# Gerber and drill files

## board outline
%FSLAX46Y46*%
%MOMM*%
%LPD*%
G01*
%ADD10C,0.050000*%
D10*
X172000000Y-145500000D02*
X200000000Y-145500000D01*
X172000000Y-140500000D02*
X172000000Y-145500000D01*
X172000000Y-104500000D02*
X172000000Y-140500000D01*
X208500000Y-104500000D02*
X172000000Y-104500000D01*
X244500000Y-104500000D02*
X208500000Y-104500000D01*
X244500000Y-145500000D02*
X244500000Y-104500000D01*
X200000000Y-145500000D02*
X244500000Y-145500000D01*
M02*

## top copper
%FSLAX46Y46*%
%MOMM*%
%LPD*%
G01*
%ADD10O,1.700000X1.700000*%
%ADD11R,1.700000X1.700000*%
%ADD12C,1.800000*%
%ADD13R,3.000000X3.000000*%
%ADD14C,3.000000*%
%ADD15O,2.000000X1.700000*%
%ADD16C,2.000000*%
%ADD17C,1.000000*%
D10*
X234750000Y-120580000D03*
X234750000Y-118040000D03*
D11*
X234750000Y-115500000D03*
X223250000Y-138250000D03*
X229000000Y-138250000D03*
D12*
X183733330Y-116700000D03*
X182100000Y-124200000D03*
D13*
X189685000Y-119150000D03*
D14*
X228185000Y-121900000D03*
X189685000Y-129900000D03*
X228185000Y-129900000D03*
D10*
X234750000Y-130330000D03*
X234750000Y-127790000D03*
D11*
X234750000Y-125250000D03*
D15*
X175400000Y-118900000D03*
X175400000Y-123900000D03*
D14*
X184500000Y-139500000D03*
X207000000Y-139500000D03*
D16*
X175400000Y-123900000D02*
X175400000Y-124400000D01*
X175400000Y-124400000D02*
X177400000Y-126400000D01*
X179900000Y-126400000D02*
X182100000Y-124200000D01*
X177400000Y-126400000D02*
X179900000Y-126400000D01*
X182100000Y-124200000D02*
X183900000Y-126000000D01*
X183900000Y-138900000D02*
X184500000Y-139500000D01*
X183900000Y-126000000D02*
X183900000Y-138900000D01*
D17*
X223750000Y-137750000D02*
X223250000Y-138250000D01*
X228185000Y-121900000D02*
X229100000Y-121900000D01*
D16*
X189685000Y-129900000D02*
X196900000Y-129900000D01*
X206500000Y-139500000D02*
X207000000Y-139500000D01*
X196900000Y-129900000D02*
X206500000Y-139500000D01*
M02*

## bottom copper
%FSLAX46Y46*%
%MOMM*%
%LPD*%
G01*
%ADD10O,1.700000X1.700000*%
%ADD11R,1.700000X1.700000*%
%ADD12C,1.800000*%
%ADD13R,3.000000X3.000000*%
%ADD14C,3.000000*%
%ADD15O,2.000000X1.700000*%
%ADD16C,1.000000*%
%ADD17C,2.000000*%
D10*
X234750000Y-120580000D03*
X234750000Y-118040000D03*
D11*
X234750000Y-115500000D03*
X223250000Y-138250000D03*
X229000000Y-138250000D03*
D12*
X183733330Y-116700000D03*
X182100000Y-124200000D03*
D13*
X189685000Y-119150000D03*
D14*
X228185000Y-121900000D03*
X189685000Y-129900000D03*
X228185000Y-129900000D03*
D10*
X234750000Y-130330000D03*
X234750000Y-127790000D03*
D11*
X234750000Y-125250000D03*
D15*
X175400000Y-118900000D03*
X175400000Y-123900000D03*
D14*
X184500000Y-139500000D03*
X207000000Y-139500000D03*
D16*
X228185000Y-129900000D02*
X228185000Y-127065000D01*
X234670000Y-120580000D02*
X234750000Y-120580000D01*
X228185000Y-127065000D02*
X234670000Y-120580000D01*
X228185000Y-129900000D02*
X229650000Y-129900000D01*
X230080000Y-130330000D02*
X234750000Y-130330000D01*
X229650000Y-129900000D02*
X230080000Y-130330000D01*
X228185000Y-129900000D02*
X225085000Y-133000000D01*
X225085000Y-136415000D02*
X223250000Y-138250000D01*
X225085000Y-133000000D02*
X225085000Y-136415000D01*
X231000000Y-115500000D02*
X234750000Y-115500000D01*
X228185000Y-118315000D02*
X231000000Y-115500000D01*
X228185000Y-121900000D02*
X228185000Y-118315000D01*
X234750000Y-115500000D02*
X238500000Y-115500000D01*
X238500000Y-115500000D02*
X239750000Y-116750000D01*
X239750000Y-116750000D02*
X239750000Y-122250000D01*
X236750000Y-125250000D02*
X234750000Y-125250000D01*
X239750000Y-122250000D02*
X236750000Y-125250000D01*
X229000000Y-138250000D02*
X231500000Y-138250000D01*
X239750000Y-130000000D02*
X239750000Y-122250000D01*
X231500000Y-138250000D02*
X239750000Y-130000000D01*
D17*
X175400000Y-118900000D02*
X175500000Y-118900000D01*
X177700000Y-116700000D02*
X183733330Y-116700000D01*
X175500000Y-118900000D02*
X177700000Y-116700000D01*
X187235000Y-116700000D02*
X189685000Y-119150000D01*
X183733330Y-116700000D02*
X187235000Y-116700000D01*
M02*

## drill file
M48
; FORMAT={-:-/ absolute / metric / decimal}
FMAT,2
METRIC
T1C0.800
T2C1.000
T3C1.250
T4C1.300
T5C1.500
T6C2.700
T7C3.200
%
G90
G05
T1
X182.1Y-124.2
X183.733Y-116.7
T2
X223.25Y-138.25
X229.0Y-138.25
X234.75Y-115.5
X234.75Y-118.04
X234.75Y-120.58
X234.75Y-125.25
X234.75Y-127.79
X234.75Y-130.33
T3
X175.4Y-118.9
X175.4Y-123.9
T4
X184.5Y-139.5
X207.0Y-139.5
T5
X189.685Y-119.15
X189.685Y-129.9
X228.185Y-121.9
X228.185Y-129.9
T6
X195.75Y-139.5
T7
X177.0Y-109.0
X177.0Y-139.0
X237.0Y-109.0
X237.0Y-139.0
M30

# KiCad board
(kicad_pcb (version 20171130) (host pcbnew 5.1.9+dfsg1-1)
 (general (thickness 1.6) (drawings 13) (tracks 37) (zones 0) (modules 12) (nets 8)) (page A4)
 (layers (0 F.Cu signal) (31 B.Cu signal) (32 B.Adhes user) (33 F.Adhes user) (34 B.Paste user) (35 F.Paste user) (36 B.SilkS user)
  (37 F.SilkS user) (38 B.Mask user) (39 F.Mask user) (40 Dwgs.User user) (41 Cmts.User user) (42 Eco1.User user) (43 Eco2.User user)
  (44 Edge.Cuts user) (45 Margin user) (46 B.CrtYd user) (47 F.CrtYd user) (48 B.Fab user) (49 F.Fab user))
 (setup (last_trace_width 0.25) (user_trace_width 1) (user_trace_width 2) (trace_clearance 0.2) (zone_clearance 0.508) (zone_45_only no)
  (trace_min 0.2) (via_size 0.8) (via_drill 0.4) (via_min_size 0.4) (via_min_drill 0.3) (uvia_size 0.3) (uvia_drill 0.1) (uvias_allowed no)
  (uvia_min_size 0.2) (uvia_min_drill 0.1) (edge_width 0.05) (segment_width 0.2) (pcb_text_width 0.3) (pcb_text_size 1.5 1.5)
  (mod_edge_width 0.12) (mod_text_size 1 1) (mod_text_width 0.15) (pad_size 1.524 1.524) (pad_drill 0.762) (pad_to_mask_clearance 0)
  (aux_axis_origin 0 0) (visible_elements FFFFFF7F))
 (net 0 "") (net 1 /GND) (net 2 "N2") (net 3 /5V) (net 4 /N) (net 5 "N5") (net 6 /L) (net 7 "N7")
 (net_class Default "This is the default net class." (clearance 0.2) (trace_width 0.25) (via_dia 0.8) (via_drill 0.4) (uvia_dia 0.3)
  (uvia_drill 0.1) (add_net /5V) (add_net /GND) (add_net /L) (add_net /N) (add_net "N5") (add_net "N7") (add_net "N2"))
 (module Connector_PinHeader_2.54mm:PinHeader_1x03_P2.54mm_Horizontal (layer F.Cu) (at 234.75 115.5)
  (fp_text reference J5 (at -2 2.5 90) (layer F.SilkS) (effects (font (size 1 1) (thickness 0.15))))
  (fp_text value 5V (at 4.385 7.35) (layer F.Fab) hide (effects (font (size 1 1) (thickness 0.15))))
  (pad 3 thru_hole oval (at 0 5.08) (size 1.7 1.7) (drill 1) (layers *.Cu *.Mask) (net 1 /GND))
  (pad 2 thru_hole oval (at 0 2.54) (size 1.7 1.7) (drill 1) (layers *.Cu *.Mask) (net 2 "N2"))
  (pad 1 thru_hole rect (at 0 0) (size 1.7 1.7) (drill 1) (layers *.Cu *.Mask) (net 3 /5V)))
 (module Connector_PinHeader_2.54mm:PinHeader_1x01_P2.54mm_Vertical (layer F.Cu) (at 223.25 138.25)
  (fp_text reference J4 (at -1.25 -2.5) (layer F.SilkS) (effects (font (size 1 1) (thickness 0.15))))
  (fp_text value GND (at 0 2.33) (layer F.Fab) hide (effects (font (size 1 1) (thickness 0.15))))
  (pad 1 thru_hole rect (at 0 0) (size 1.7 1.7) (drill 1) (layers *.Cu *.Mask) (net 1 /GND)))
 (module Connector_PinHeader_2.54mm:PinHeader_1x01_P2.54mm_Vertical (layer F.Cu) (at 229 138.25)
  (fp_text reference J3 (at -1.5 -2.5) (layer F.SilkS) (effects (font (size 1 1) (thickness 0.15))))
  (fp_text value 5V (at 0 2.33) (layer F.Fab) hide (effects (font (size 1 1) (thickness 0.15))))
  (pad 1 thru_hole rect (at 0 0) (size 1.7 1.7) (drill 1) (layers *.Cu *.Mask) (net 3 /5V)))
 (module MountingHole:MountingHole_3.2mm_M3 (layer F.Cu) (at 237 109)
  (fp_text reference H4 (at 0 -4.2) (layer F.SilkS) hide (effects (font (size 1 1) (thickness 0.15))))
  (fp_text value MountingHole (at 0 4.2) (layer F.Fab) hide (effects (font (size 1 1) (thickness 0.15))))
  (pad 1 np_thru_hole circle (at 0 0) (size 3.2 3.2) (drill 3.2) (layers *.Cu *.Mask)))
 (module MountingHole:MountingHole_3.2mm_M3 (layer F.Cu) (at 237 139)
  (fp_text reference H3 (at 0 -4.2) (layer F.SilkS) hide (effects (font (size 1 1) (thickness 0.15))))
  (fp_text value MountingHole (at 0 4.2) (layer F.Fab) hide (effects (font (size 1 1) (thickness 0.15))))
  (pad 1 np_thru_hole circle (at 0 0) (size 3.2 3.2) (drill 3.2) (layers *.Cu *.Mask)))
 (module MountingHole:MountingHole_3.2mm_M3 (layer F.Cu) (at 177 109)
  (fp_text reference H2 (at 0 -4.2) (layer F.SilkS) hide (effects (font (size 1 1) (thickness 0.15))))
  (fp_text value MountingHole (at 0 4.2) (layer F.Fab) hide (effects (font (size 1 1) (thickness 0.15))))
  (pad 1 np_thru_hole circle (at 0 0) (size 3.2 3.2) (drill 3.2) (layers *.Cu *.Mask)))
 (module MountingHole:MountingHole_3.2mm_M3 (layer F.Cu) (at 177 139)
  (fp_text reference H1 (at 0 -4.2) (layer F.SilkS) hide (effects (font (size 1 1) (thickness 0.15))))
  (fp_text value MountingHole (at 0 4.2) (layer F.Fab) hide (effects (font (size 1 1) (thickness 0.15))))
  (pad 1 np_thru_hole circle (at 0 0) (size 3.2 3.2) (drill 3.2) (layers *.Cu *.Mask)))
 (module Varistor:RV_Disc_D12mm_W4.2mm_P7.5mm (layer F.Cu) (at 182.1 124.2 90)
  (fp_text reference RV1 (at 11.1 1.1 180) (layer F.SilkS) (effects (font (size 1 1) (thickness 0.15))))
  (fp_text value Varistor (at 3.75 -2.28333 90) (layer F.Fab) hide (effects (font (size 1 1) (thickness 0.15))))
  (pad 2 thru_hole circle (at 7.5 1.63333 90) (size 1.8 1.8) (drill 0.8) (layers *.Cu *.Mask) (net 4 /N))
  (pad 1 thru_hole circle (at 0 0 90) (size 1.8 1.8) (drill 0.8) (layers *.Cu *.Mask) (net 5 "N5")))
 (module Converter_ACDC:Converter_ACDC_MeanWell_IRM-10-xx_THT (layer F.Cu) (at 189.685 119.15)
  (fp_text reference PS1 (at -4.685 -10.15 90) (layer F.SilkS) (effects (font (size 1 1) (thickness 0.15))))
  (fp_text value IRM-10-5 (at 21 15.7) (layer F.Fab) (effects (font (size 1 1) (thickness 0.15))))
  (pad 1 thru_hole rect (at 0 0) (size 3 3) (drill 1.5) (layers *.Cu *.Mask) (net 4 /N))
  (pad 4 thru_hole circle (at 38.5 2.75) (size 3 3) (drill 1.5) (layers *.Cu *.Mask) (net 3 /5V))
  (pad 2 thru_hole circle (at 0 10.75) (size 3 3) (drill 1.5) (layers *.Cu *.Mask) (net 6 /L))
  (pad 3 thru_hole circle (at 38.5 10.75) (size 3 3) (drill 1.5) (layers *.Cu *.Mask) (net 1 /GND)))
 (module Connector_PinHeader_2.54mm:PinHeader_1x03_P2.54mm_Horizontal (layer F.Cu) (at 234.75 125.25)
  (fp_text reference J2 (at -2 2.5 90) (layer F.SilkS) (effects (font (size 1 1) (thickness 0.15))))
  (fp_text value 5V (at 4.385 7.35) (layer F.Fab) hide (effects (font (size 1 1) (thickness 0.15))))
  (pad 3 thru_hole oval (at 0 5.08) (size 1.7 1.7) (drill 1) (layers *.Cu *.Mask) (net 1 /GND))
  (pad 2 thru_hole oval (at 0 2.54) (size 1.7 1.7) (drill 1) (layers *.Cu *.Mask) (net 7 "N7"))
  (pad 1 thru_hole rect (at 0 0) (size 1.7 1.7) (drill 1) (layers *.Cu *.Mask) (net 3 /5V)))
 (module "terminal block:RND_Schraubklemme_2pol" (layer F.Cu) (at 175.4 118.9 270)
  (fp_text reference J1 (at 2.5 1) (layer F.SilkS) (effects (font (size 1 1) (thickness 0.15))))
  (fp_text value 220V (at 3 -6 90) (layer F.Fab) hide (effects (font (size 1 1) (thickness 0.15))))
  (pad 1 thru_hole oval (at 0 0 270) (size 1.7 2) (drill 1.25) (layers *.Cu *.Mask) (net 4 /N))
  (pad 2 thru_hole oval (at 5 0 270) (size 1.7 2) (drill 1.25) (layers *.Cu *.Mask) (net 5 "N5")))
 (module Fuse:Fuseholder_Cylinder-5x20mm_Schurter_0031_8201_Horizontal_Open (layer F.Cu) (at 207 139.5 180)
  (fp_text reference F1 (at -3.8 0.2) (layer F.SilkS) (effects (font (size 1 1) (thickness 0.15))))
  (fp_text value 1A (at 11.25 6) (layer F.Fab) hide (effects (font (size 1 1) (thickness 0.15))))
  (pad "" np_thru_hole circle (at 11.25 0 180) (size 2.7 2.7) (drill 2.7) (layers *.Cu *.Mask))
  (pad 2 thru_hole circle (at 22.5 0 180) (size 3 3) (drill 1.3) (layers *.Cu *.Mask) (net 5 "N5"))
  (pad 1 thru_hole circle (at 0 0 180) (size 3 3) (drill 1.3) (layers *.Cu *.Mask) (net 6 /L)))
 (gr_line (start 172 145.5) (end 200 145.5) (layer Edge.Cuts) (width 0.05))
 (gr_line (start 172 140.5) (end 172 145.5) (layer Edge.Cuts) (width 0.05))
 (gr_line (start 172 104.5) (end 172 140.5) (layer Edge.Cuts) (width 0.05))
 (gr_line (start 208.5 104.5) (end 172 104.5) (layer Edge.Cuts) (width 0.05))
 (gr_line (start 244.5 104.5) (end 208.5 104.5) (layer Edge.Cuts) (width 0.05))
 (gr_line (start 244.5 145.5) (end 244.5 104.5) (layer Edge.Cuts) (width 0.05))
 (gr_line (start 200 145.5) (end 244.5 145.5) (layer Edge.Cuts) (width 0.05))
 (segment (start 175.4 123.9) (end 175.4 124.4) (width 2) (layer F.Cu) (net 5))
 (segment (start 175.4 124.4) (end 177.4 126.4) (width 2) (layer F.Cu) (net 5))
 (segment (start 179.9 126.4) (end 182.1 124.2) (width 2) (layer F.Cu) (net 5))
 (segment (start 177.4 126.4) (end 179.9 126.4) (width 2) (layer F.Cu) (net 5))
 (segment (start 182.1 124.2) (end 183.9 126) (width 2) (layer F.Cu) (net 5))
 (segment (start 183.9 138.9) (end 184.5 139.5) (width 2) (layer F.Cu) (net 5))
 (segment (start 183.9 126) (end 183.9 138.9) (width 2) (layer F.Cu) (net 5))
 (segment (start 223.75 137.75) (end 223.25 138.25) (width 1) (layer F.Cu) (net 1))
 (segment (start 228.185 129.9) (end 228.185 127.065) (width 1) (layer B.Cu) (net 1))
 (segment (start 234.67 120.58) (end 234.75 120.58) (width 1) (layer B.Cu) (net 1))
 (segment (start 228.185 127.065) (end 234.67 120.58) (width 1) (layer B.Cu) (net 1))
 (segment (start 228.185 129.9) (end 229.65 129.9) (width 1) (layer B.Cu) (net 1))
 (segment (start 230.08 130.33) (end 234.75 130.33) (width 1) (layer B.Cu) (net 1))
 (segment (start 229.65 129.9) (end 230.08 130.33) (width 1) (layer B.Cu) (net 1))
 (segment (start 228.185 129.9) (end 225.085 133) (width 1) (layer B.Cu) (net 1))
 (segment (start 225.085 136.415) (end 223.25 138.25) (width 1) (layer B.Cu) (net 1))
 (segment (start 225.085 133) (end 225.085 136.415) (width 1) (layer B.Cu) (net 1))
 (segment (start 228.185 121.9) (end 229.1 121.9) (width 1) (layer F.Cu) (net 3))
 (segment (start 231 115.5) (end 234.75 115.5) (width 1) (layer B.Cu) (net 3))
 (segment (start 228.185 118.315) (end 231 115.5) (width 1) (layer B.Cu) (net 3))
 (segment (start 228.185 121.9) (end 228.185 118.315) (width 1) (layer B.Cu) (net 3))
 (segment (start 234.75 115.5) (end 238.5 115.5) (width 1) (layer B.Cu) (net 3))
 (segment (start 238.5 115.5) (end 239.75 116.75) (width 1) (layer B.Cu) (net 3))
 (segment (start 239.75 116.75) (end 239.75 122.25) (width 1) (layer B.Cu) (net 3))
 (segment (start 236.75 125.25) (end 234.75 125.25) (width 1) (layer B.Cu) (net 3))
 (segment (start 239.75 122.25) (end 236.75 125.25) (width 1) (layer B.Cu) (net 3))
 (segment (start 229 138.25) (end 231.5 138.25) (width 1) (layer B.Cu) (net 3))
 (segment (start 239.75 130) (end 239.75 122.25) (width 1) (layer B.Cu) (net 3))
 (segment (start 231.5 138.25) (end 239.75 130) (width 1) (layer B.Cu) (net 3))
 (segment (start 189.685 129.9) (end 196.9 129.9) (width 2) (layer F.Cu) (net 6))
 (segment (start 206.5 139.5) (end 207 139.5) (width 2) (layer F.Cu) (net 6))
 (segment (start 196.9 129.9) (end 206.5 139.5) (width 2) (layer F.Cu) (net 6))
 (segment (start 175.4 118.9) (end 175.5 118.9) (width 2) (layer B.Cu) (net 4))
 (segment (start 177.7 116.7) (end 183.73333 116.7) (width 2) (layer B.Cu) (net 4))
 (segment (start 175.5 118.9) (end 177.7 116.7) (width 2) (layer B.Cu) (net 4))
 (segment (start 187.235 116.7) (end 189.685 119.15) (width 2) (layer B.Cu) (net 4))
 (segment (start 183.73333 116.7) (end 187.235 116.7) (width 2) (layer B.Cu) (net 4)))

